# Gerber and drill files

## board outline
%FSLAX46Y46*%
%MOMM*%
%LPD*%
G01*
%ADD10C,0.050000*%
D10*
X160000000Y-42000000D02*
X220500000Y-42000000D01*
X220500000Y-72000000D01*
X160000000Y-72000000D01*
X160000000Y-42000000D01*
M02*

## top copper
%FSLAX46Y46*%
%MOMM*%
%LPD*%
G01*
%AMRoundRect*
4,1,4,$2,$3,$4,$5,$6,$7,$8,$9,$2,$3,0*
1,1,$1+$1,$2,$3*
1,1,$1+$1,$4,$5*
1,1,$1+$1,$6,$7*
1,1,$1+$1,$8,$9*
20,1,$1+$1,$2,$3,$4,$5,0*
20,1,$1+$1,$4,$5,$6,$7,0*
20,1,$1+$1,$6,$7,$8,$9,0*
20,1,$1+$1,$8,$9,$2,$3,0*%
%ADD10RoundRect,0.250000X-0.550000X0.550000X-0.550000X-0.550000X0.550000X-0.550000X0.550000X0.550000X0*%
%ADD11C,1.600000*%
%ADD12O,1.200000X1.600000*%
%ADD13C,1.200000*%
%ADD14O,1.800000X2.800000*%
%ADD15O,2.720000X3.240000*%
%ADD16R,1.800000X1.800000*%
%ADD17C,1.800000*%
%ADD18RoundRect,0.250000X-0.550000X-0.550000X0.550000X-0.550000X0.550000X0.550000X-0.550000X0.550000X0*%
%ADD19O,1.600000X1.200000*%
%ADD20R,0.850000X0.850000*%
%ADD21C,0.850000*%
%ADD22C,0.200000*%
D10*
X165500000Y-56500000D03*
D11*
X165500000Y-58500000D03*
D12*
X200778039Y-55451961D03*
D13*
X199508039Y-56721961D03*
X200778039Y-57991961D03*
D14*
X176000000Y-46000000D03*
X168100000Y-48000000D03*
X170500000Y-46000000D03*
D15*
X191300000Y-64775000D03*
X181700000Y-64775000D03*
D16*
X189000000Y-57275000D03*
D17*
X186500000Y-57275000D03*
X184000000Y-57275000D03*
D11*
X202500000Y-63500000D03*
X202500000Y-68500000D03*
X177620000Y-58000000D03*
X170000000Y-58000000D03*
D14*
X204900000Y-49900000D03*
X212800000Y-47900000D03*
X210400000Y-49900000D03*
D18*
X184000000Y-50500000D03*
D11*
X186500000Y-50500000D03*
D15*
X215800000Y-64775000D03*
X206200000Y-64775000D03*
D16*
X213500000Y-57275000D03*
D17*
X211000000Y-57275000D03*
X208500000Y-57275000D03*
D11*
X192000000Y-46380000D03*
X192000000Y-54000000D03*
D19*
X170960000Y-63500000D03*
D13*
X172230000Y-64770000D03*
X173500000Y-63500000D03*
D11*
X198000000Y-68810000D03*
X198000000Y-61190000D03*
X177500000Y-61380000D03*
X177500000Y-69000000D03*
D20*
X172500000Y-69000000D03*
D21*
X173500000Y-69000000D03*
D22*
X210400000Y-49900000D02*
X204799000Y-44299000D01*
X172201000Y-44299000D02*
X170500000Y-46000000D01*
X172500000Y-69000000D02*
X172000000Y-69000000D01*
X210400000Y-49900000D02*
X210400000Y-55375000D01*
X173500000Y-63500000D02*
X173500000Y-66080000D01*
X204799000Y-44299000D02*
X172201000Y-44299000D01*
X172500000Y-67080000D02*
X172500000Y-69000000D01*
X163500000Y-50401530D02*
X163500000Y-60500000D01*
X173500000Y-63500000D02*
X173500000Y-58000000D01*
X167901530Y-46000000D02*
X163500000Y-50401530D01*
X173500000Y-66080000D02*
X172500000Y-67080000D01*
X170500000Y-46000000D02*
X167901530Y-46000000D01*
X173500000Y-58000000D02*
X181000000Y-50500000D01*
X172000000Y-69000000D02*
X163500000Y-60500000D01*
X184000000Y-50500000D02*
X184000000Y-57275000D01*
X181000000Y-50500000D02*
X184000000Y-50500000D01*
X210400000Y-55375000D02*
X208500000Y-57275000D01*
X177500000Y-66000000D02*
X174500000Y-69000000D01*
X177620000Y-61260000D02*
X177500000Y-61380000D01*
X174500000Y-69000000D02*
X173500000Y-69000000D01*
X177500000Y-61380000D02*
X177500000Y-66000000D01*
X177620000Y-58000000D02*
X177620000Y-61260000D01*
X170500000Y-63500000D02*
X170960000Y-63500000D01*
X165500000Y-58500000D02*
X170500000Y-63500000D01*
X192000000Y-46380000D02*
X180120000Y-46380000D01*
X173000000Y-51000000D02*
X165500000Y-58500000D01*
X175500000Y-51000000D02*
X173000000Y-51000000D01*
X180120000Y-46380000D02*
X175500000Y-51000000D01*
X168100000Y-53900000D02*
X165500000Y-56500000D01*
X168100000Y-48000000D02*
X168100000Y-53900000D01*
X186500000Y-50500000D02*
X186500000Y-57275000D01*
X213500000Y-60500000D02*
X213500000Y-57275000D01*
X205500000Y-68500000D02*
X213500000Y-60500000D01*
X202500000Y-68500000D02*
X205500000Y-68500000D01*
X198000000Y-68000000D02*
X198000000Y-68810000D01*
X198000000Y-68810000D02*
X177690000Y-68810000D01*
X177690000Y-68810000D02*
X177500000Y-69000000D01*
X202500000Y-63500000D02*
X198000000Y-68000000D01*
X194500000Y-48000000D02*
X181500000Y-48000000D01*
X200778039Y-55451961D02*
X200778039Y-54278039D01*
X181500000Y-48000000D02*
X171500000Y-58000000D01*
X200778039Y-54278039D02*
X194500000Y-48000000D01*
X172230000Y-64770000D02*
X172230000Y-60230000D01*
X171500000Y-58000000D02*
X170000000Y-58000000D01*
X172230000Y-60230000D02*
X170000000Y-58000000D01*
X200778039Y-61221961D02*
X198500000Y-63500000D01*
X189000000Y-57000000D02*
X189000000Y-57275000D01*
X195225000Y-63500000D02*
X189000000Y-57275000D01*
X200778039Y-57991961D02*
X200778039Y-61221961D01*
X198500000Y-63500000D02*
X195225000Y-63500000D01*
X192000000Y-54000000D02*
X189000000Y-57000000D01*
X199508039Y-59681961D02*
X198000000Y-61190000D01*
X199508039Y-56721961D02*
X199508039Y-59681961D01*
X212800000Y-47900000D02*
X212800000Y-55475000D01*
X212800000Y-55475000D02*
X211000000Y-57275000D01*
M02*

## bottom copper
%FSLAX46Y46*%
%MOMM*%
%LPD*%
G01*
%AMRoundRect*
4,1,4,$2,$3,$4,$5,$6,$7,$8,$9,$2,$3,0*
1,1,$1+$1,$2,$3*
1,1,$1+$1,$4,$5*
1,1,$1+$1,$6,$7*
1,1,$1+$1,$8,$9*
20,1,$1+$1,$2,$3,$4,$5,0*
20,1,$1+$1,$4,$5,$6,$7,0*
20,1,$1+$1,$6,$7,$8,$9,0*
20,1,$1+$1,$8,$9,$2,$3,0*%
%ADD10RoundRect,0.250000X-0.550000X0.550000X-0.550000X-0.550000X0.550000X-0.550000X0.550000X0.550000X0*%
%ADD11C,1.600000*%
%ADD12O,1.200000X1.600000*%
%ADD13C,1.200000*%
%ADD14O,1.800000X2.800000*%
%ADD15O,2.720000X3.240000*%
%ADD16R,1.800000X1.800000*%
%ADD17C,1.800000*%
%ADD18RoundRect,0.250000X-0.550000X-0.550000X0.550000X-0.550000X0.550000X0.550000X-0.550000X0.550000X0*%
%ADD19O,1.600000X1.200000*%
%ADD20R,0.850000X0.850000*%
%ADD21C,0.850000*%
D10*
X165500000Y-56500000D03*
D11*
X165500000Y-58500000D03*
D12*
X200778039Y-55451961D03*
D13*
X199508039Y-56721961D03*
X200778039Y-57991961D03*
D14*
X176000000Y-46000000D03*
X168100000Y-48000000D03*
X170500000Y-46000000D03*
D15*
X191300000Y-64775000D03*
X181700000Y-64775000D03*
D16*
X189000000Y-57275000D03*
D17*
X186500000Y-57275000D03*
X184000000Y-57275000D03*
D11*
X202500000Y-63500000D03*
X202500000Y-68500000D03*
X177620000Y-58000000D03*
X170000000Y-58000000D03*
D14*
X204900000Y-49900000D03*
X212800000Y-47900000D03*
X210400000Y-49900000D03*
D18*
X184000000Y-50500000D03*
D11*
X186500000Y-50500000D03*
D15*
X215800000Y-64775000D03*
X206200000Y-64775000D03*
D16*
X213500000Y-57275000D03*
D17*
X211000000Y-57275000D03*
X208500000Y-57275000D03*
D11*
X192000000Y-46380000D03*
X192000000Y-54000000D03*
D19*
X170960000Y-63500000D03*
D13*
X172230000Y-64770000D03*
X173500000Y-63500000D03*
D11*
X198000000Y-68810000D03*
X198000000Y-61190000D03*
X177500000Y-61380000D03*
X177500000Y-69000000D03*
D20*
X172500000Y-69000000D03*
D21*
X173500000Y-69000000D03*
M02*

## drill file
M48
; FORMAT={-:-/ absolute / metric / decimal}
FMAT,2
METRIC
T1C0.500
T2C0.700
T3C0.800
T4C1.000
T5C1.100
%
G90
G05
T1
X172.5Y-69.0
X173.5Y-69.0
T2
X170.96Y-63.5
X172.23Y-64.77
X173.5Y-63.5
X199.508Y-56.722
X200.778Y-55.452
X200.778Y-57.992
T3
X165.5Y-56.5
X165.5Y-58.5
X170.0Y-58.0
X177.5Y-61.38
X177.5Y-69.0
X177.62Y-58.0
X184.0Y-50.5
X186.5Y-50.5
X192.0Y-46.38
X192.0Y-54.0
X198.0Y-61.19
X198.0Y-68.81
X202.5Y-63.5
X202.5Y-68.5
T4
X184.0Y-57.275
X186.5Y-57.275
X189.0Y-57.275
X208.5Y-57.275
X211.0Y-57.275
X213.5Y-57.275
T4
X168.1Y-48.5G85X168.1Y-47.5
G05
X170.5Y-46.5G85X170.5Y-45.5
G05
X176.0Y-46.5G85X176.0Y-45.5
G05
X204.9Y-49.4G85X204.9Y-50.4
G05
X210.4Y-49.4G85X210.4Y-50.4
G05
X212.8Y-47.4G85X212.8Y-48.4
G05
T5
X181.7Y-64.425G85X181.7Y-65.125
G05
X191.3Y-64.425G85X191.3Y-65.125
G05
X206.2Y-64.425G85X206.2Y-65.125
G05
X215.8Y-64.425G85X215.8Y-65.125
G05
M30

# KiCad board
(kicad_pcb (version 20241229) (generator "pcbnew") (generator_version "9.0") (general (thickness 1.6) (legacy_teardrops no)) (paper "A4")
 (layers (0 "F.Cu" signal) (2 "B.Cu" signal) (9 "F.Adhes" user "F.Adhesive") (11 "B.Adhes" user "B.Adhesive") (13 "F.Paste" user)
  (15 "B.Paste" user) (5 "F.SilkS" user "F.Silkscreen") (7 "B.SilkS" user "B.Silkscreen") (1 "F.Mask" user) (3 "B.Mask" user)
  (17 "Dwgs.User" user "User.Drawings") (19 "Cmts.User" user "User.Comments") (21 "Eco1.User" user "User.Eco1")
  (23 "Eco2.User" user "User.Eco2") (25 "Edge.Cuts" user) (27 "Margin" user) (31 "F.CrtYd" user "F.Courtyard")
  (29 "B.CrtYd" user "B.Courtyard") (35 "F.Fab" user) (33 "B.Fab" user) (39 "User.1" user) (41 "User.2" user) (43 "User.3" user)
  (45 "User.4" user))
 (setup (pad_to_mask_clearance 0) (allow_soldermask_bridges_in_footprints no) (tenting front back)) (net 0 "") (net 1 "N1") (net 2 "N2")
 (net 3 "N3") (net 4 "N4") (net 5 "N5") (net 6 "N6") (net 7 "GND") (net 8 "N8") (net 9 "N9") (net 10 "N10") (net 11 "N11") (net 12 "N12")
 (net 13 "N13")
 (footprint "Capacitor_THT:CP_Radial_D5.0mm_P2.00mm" (layer "F.Cu") (at 165.5 56.5 -90)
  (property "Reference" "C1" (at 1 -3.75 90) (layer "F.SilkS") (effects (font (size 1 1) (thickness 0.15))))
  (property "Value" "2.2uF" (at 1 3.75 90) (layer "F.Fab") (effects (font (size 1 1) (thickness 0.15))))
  (pad "1" thru_hole roundrect (at 0 0 270) (size 1.6 1.6) (drill 0.8) (layers "*.Cu" "*.Mask") (remove_unused_layers no)
   (roundrect_rratio 0.15625) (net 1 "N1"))
  (pad "2" thru_hole circle (at 2 0 270) (size 1.6 1.6) (drill 0.8) (layers "*.Cu" "*.Mask") (remove_unused_layers no) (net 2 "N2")))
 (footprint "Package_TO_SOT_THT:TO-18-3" (layer "F.Cu") (at 200.778039 55.451961 -90)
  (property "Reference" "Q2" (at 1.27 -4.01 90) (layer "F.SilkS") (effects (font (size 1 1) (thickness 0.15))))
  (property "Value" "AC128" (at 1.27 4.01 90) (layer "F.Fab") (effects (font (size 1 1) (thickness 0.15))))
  (pad "1" thru_hole oval (at 0 0 270) (size 1.6 1.2) (drill 0.7) (layers "*.Cu" "*.Mask") (remove_unused_layers no) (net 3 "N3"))
  (pad "2" thru_hole circle (at 1.27 1.27 270) (size 1.2 1.2) (drill 0.7) (layers "*.Cu" "*.Mask") (remove_unused_layers no) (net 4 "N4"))
  (pad "3" thru_hole circle (at 2.54 0 270) (size 1.2 1.2) (drill 0.7) (layers "*.Cu" "*.Mask") (remove_unused_layers no) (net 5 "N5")))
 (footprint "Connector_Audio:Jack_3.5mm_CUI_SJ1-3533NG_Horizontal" (layer "F.Cu") (at 168.1 48 90)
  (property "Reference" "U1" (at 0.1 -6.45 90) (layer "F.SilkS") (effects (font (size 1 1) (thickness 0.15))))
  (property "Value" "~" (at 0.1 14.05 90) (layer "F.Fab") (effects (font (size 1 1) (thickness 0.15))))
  (pad "R" thru_hole oval (at 2 7.9 90) (size 2.8 1.8) (drill oval 2 1) (layers "*.Cu" "*.Mask") (remove_unused_layers no) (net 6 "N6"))
  (pad "S" thru_hole oval (at 0 0 90) (size 2.8 1.8) (drill oval 2 1) (layers "*.Cu" "*.Mask") (remove_unused_layers no) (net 1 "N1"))
  (pad "T" thru_hole oval (at 2 2.4 90) (size 2.8 1.8) (drill oval 2 1) (layers "*.Cu" "*.Mask") (remove_unused_layers no) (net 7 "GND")))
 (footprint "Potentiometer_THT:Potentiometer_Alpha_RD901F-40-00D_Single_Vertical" (layer "F.Cu") (at 189 57.275 -90)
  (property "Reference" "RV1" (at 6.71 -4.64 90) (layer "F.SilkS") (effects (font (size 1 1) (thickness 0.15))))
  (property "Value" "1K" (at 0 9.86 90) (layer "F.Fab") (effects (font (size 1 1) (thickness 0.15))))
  (pad "" thru_hole oval (at 7.5 -2.3) (size 2.72 3.24) (drill oval 1.1 1.8) (layers "*.Cu" "*.Mask") (remove_unused_layers no))
  (pad "" thru_hole oval (at 7.5 7.3) (size 2.72 3.24) (drill oval 1.1 1.8) (layers "*.Cu" "*.Mask") (remove_unused_layers no))
  (pad "1" thru_hole rect (at 0 0) (size 1.8 1.8) (drill 1) (layers "*.Cu" "*.Mask") (remove_unused_layers no) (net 5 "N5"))
  (pad "2" thru_hole circle (at 0 2.5) (size 1.8 1.8) (drill 1) (layers "*.Cu" "*.Mask") (remove_unused_layers no) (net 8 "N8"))
  (pad "3" thru_hole circle (at 0 5) (size 1.8 1.8) (drill 1) (layers "*.Cu" "*.Mask") (remove_unused_layers no) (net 7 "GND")))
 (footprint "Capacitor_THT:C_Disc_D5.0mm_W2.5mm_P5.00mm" (layer "F.Cu") (at 202.5 63.5 -90)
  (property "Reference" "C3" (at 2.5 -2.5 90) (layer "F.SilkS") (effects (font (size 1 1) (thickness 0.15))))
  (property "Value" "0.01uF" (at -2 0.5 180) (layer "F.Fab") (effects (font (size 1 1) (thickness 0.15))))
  (pad "1" thru_hole circle (at 0 0 270) (size 1.6 1.6) (drill 0.8) (layers "*.Cu" "*.Mask") (remove_unused_layers no) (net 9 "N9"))
  (pad "2" thru_hole circle (at 5 0 270) (size 1.6 1.6) (drill 0.8) (layers "*.Cu" "*.Mask") (remove_unused_layers no) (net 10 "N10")))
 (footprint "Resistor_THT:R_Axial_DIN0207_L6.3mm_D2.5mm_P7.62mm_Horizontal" (layer "F.Cu") (at 177.62 58 180)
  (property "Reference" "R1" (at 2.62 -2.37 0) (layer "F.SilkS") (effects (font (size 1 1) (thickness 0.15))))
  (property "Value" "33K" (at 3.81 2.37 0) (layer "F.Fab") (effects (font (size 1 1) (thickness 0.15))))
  (pad "1" thru_hole circle (at 0 0 180) (size 1.6 1.6) (drill 0.8) (layers "*.Cu" "*.Mask") (remove_unused_layers no) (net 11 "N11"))
  (pad "2" thru_hole circle (at 7.62 0 180) (size 1.6 1.6) (drill 0.8) (layers "*.Cu" "*.Mask") (remove_unused_layers no) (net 3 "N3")))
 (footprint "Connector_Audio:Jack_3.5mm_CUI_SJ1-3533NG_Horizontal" (layer "F.Cu") (at 212.8 47.9 -90)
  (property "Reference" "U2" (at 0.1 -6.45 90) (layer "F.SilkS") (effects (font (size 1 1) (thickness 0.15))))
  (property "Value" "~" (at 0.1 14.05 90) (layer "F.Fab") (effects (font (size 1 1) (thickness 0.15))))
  (pad "R" thru_hole oval (at 2 7.9 270) (size 2.8 1.8) (drill oval 2 1) (layers "*.Cu" "*.Mask") (remove_unused_layers no) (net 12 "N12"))
  (pad "S" thru_hole oval (at 0 0 270) (size 2.8 1.8) (drill oval 2 1) (layers "*.Cu" "*.Mask") (remove_unused_layers no) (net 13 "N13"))
  (pad "T" thru_hole oval (at 2 2.4 270) (size 2.8 1.8) (drill oval 2 1) (layers "*.Cu" "*.Mask") (remove_unused_layers no) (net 7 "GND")))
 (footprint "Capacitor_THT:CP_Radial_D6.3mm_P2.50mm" (layer "F.Cu") (at 184 50.5)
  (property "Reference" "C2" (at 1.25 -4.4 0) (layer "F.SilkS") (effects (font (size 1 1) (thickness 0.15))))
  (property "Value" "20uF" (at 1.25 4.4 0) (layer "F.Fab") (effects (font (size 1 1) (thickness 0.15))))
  (pad "1" thru_hole roundrect (at 0 0) (size 1.6 1.6) (drill 0.8) (layers "*.Cu" "*.Mask") (remove_unused_layers no)
   (roundrect_rratio 0.15625) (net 7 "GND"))
  (pad "2" thru_hole circle (at 2.5 0) (size 1.6 1.6) (drill 0.8) (layers "*.Cu" "*.Mask") (remove_unused_layers no) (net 8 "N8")))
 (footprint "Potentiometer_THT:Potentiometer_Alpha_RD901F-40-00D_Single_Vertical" (layer "F.Cu") (at 213.5 57.275 -90)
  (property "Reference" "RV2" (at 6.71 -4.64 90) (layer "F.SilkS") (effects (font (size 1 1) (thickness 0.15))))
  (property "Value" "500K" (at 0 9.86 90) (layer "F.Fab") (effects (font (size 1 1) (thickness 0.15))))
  (pad "" thru_hole oval (at 7.5 -2.3) (size 2.72 3.24) (drill oval 1.1 1.8) (layers "*.Cu" "*.Mask") (remove_unused_layers no))
  (pad "" thru_hole oval (at 7.5 7.3) (size 2.72 3.24) (drill oval 1.1 1.8) (layers "*.Cu" "*.Mask") (remove_unused_layers no))
  (pad "1" thru_hole rect (at 0 0) (size 1.8 1.8) (drill 1) (layers "*.Cu" "*.Mask") (remove_unused_layers no) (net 10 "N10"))
  (pad "2" thru_hole circle (at 0 2.5) (size 1.8 1.8) (drill 1) (layers "*.Cu" "*.Mask") (remove_unused_layers no) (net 13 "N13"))
  (pad "3" thru_hole circle (at 0 5) (size 1.8 1.8) (drill 1) (layers "*.Cu" "*.Mask") (remove_unused_layers no) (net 7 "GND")))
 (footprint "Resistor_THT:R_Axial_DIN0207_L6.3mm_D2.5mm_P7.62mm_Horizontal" (layer "F.Cu") (at 192 46.38 -90)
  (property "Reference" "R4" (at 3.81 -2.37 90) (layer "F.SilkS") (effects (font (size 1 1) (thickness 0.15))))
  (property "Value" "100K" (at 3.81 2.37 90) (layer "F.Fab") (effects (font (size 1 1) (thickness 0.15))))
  (pad "1" thru_hole circle (at 0 0 270) (size 1.6 1.6) (drill 0.8) (layers "*.Cu" "*.Mask") (remove_unused_layers no) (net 2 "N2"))
  (pad "2" thru_hole circle (at 7.62 0 270) (size 1.6 1.6) (drill 0.8) (layers "*.Cu" "*.Mask") (remove_unused_layers no) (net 5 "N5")))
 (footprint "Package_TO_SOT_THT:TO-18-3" (layer "F.Cu") (at 170.96 63.5)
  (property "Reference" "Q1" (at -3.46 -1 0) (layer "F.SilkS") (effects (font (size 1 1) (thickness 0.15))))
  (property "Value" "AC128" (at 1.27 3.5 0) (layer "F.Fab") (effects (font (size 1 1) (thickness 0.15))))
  (pad "1" thru_hole oval (at 0 0) (size 1.6 1.2) (drill 0.7) (layers "*.Cu" "*.Mask") (remove_unused_layers no) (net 2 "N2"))
  (pad "2" thru_hole circle (at 1.27 1.27) (size 1.2 1.2) (drill 0.7) (layers "*.Cu" "*.Mask") (remove_unused_layers no) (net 3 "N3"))
  (pad "3" thru_hole circle (at 2.54 0) (size 1.2 1.2) (drill 0.7) (layers "*.Cu" "*.Mask") (remove_unused_layers no) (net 7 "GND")))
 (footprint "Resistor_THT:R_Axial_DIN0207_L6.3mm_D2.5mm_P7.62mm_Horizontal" (layer "F.Cu") (at 198 68.81 90)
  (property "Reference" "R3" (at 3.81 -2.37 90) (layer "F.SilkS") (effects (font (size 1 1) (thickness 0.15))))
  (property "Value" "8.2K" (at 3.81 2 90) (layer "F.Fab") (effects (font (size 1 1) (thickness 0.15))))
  (pad "1" thru_hole circle (at 0 0 90) (size 1.6 1.6) (drill 0.8) (layers "*.Cu" "*.Mask") (remove_unused_layers no) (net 9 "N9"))
  (pad "2" thru_hole circle (at 7.62 0 90) (size 1.6 1.6) (drill 0.8) (layers "*.Cu" "*.Mask") (remove_unused_layers no) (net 4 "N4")))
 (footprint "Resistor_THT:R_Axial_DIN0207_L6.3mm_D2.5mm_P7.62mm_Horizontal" (layer "F.Cu") (at 177.5 61.38 -90)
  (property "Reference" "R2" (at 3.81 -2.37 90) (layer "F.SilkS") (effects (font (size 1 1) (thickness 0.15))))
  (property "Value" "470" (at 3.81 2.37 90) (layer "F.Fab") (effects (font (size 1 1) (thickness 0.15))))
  (pad "1" thru_hole circle (at 0 0 270) (size 1.6 1.6) (drill 0.8) (layers "*.Cu" "*.Mask") (remove_unused_layers no) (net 11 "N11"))
  (pad "2" thru_hole circle (at 7.62 0 270) (size 1.6 1.6) (drill 0.8) (layers "*.Cu" "*.Mask") (remove_unused_layers no) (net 9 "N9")))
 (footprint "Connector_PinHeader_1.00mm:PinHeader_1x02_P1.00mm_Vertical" (layer "F.Cu") (at 172.5 69 90)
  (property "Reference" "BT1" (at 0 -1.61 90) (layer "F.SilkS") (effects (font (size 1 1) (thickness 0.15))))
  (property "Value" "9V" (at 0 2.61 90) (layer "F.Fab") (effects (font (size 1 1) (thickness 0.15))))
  (pad "1" thru_hole rect (at 0 0 90) (size 0.85 0.85) (drill 0.5) (layers "*.Cu" "*.Mask") (remove_unused_layers no) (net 7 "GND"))
  (pad "2" thru_hole circle (at 0 1 90) (size 0.85 0.85) (drill 0.5) (layers "*.Cu" "*.Mask") (remove_unused_layers no) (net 11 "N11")))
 (gr_poly (pts (xy 160 42) (xy 220.5 42) (xy 220.5 72) (xy 160 72)) (stroke (width 0.05) (type solid)) (fill no) (layer "Edge.Cuts"))
 (segment (start 210.4 49.9) (end 204.799 44.299) (width 0.2) (layer "F.Cu") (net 7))
 (segment (start 172.201 44.299) (end 170.5 46) (width 0.2) (layer "F.Cu") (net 7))
 (segment (start 172.5 69) (end 172 69) (width 0.2) (layer "F.Cu") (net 7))
 (segment (start 210.4 49.9) (end 210.4 55.375) (width 0.2) (layer "F.Cu") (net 7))
 (segment (start 173.5 63.5) (end 173.5 66.08) (width 0.2) (layer "F.Cu") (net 7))
 (segment (start 204.799 44.299) (end 172.201 44.299) (width 0.2) (layer "F.Cu") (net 7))
 (segment (start 172.5 67.08) (end 172.5 69) (width 0.2) (layer "F.Cu") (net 7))
 (segment (start 163.5 50.40153) (end 163.5 60.5) (width 0.2) (layer "F.Cu") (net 7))
 (segment (start 173.5 63.5) (end 173.5 58) (width 0.2) (layer "F.Cu") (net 7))
 (segment (start 167.90153 46) (end 163.5 50.40153) (width 0.2) (layer "F.Cu") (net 7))
 (segment (start 173.5 66.08) (end 172.5 67.08) (width 0.2) (layer "F.Cu") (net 7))
 (segment (start 170.5 46) (end 167.90153 46) (width 0.2) (layer "F.Cu") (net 7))
 (segment (start 173.5 58) (end 181 50.5) (width 0.2) (layer "F.Cu") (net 7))
 (segment (start 172 69) (end 163.5 60.5) (width 0.2) (layer "F.Cu") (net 7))
 (segment (start 184 50.5) (end 184 57.275) (width 0.2) (layer "F.Cu") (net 7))
 (segment (start 181 50.5) (end 184 50.5) (width 0.2) (layer "F.Cu") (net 7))
 (segment (start 210.4 55.375) (end 208.5 57.275) (width 0.2) (layer "F.Cu") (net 7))
 (segment (start 177.5 66) (end 174.5 69) (width 0.2) (layer "F.Cu") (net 11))
 (segment (start 177.62 61.26) (end 177.5 61.38) (width 0.2) (layer "F.Cu") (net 11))
 (segment (start 174.5 69) (end 173.5 69) (width 0.2) (layer "F.Cu") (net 11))
 (segment (start 177.5 61.38) (end 177.5 66) (width 0.2) (layer "F.Cu") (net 11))
 (segment (start 177.62 58) (end 177.62 61.26) (width 0.2) (layer "F.Cu") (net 11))
 (segment (start 170.5 63.5) (end 170.96 63.5) (width 0.2) (layer "F.Cu") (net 2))
 (segment (start 165.5 58.5) (end 170.5 63.5) (width 0.2) (layer "F.Cu") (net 2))
 (segment (start 192 46.38) (end 180.12 46.38) (width 0.2) (layer "F.Cu") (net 2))
 (segment (start 173 51) (end 165.5 58.5) (width 0.2) (layer "F.Cu") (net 2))
 (segment (start 175.5 51) (end 173 51) (width 0.2) (layer "F.Cu") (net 2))
 (segment (start 180.12 46.38) (end 175.5 51) (width 0.2) (layer "F.Cu") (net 2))
 (segment (start 168.1 53.9) (end 165.5 56.5) (width 0.2) (layer "F.Cu") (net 1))
 (segment (start 168.1 48) (end 168.1 53.9) (width 0.2) (layer "F.Cu") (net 1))
 (segment (start 186.5 50.5) (end 186.5 57.275) (width 0.2) (layer "F.Cu") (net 8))
 (segment (start 213.5 60.5) (end 213.5 57.275) (width 0.2) (layer "F.Cu") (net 10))
 (segment (start 205.5 68.5) (end 213.5 60.5) (width 0.2) (layer "F.Cu") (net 10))
 (segment (start 202.5 68.5) (end 205.5 68.5) (width 0.2) (layer "F.Cu") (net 10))
 (segment (start 198 68) (end 198 68.81) (width 0.2) (layer "F.Cu") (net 9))
 (segment (start 198 68.81) (end 177.69 68.81) (width 0.2) (layer "F.Cu") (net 9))
 (segment (start 177.69 68.81) (end 177.5 69) (width 0.2) (layer "F.Cu") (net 9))
 (segment (start 202.5 63.5) (end 198 68) (width 0.2) (layer "F.Cu") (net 9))
 (segment (start 194.5 48) (end 181.5 48) (width 0.2) (layer "F.Cu") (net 3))
 (segment (start 200.778039 55.451961) (end 200.778039 54.278039) (width 0.2) (layer "F.Cu") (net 3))
 (segment (start 181.5 48) (end 171.5 58) (width 0.2) (layer "F.Cu") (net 3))
 (segment (start 200.778039 54.278039) (end 194.5 48) (width 0.2) (layer "F.Cu") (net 3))
 (segment (start 172.23 64.77) (end 172.23 60.23) (width 0.2) (layer "F.Cu") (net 3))
 (segment (start 171.5 58) (end 170 58) (width 0.2) (layer "F.Cu") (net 3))
 (segment (start 172.23 60.23) (end 170 58) (width 0.2) (layer "F.Cu") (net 3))
 (segment (start 200.778039 61.221961) (end 198.5 63.5) (width 0.2) (layer "F.Cu") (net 5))
 (segment (start 189 57) (end 189 57.275) (width 0.2) (layer "F.Cu") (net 5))
 (segment (start 195.225 63.5) (end 189 57.275) (width 0.2) (layer "F.Cu") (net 5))
 (segment (start 200.778039 57.991961) (end 200.778039 61.221961) (width 0.2) (layer "F.Cu") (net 5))
 (segment (start 198.5 63.5) (end 195.225 63.5) (width 0.2) (layer "F.Cu") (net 5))
 (segment (start 192 54) (end 189 57) (width 0.2) (layer "F.Cu") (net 5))
 (segment (start 199.508039 59.681961) (end 198 61.19) (width 0.2) (layer "F.Cu") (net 4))
 (segment (start 199.508039 56.721961) (end 199.508039 59.681961) (width 0.2) (layer "F.Cu") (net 4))
 (segment (start 212.8 47.9) (end 212.8 55.475) (width 0.2) (layer "F.Cu") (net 13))
 (segment (start 212.8 55.475) (end 211 57.275) (width 0.2) (layer "F.Cu") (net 13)))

